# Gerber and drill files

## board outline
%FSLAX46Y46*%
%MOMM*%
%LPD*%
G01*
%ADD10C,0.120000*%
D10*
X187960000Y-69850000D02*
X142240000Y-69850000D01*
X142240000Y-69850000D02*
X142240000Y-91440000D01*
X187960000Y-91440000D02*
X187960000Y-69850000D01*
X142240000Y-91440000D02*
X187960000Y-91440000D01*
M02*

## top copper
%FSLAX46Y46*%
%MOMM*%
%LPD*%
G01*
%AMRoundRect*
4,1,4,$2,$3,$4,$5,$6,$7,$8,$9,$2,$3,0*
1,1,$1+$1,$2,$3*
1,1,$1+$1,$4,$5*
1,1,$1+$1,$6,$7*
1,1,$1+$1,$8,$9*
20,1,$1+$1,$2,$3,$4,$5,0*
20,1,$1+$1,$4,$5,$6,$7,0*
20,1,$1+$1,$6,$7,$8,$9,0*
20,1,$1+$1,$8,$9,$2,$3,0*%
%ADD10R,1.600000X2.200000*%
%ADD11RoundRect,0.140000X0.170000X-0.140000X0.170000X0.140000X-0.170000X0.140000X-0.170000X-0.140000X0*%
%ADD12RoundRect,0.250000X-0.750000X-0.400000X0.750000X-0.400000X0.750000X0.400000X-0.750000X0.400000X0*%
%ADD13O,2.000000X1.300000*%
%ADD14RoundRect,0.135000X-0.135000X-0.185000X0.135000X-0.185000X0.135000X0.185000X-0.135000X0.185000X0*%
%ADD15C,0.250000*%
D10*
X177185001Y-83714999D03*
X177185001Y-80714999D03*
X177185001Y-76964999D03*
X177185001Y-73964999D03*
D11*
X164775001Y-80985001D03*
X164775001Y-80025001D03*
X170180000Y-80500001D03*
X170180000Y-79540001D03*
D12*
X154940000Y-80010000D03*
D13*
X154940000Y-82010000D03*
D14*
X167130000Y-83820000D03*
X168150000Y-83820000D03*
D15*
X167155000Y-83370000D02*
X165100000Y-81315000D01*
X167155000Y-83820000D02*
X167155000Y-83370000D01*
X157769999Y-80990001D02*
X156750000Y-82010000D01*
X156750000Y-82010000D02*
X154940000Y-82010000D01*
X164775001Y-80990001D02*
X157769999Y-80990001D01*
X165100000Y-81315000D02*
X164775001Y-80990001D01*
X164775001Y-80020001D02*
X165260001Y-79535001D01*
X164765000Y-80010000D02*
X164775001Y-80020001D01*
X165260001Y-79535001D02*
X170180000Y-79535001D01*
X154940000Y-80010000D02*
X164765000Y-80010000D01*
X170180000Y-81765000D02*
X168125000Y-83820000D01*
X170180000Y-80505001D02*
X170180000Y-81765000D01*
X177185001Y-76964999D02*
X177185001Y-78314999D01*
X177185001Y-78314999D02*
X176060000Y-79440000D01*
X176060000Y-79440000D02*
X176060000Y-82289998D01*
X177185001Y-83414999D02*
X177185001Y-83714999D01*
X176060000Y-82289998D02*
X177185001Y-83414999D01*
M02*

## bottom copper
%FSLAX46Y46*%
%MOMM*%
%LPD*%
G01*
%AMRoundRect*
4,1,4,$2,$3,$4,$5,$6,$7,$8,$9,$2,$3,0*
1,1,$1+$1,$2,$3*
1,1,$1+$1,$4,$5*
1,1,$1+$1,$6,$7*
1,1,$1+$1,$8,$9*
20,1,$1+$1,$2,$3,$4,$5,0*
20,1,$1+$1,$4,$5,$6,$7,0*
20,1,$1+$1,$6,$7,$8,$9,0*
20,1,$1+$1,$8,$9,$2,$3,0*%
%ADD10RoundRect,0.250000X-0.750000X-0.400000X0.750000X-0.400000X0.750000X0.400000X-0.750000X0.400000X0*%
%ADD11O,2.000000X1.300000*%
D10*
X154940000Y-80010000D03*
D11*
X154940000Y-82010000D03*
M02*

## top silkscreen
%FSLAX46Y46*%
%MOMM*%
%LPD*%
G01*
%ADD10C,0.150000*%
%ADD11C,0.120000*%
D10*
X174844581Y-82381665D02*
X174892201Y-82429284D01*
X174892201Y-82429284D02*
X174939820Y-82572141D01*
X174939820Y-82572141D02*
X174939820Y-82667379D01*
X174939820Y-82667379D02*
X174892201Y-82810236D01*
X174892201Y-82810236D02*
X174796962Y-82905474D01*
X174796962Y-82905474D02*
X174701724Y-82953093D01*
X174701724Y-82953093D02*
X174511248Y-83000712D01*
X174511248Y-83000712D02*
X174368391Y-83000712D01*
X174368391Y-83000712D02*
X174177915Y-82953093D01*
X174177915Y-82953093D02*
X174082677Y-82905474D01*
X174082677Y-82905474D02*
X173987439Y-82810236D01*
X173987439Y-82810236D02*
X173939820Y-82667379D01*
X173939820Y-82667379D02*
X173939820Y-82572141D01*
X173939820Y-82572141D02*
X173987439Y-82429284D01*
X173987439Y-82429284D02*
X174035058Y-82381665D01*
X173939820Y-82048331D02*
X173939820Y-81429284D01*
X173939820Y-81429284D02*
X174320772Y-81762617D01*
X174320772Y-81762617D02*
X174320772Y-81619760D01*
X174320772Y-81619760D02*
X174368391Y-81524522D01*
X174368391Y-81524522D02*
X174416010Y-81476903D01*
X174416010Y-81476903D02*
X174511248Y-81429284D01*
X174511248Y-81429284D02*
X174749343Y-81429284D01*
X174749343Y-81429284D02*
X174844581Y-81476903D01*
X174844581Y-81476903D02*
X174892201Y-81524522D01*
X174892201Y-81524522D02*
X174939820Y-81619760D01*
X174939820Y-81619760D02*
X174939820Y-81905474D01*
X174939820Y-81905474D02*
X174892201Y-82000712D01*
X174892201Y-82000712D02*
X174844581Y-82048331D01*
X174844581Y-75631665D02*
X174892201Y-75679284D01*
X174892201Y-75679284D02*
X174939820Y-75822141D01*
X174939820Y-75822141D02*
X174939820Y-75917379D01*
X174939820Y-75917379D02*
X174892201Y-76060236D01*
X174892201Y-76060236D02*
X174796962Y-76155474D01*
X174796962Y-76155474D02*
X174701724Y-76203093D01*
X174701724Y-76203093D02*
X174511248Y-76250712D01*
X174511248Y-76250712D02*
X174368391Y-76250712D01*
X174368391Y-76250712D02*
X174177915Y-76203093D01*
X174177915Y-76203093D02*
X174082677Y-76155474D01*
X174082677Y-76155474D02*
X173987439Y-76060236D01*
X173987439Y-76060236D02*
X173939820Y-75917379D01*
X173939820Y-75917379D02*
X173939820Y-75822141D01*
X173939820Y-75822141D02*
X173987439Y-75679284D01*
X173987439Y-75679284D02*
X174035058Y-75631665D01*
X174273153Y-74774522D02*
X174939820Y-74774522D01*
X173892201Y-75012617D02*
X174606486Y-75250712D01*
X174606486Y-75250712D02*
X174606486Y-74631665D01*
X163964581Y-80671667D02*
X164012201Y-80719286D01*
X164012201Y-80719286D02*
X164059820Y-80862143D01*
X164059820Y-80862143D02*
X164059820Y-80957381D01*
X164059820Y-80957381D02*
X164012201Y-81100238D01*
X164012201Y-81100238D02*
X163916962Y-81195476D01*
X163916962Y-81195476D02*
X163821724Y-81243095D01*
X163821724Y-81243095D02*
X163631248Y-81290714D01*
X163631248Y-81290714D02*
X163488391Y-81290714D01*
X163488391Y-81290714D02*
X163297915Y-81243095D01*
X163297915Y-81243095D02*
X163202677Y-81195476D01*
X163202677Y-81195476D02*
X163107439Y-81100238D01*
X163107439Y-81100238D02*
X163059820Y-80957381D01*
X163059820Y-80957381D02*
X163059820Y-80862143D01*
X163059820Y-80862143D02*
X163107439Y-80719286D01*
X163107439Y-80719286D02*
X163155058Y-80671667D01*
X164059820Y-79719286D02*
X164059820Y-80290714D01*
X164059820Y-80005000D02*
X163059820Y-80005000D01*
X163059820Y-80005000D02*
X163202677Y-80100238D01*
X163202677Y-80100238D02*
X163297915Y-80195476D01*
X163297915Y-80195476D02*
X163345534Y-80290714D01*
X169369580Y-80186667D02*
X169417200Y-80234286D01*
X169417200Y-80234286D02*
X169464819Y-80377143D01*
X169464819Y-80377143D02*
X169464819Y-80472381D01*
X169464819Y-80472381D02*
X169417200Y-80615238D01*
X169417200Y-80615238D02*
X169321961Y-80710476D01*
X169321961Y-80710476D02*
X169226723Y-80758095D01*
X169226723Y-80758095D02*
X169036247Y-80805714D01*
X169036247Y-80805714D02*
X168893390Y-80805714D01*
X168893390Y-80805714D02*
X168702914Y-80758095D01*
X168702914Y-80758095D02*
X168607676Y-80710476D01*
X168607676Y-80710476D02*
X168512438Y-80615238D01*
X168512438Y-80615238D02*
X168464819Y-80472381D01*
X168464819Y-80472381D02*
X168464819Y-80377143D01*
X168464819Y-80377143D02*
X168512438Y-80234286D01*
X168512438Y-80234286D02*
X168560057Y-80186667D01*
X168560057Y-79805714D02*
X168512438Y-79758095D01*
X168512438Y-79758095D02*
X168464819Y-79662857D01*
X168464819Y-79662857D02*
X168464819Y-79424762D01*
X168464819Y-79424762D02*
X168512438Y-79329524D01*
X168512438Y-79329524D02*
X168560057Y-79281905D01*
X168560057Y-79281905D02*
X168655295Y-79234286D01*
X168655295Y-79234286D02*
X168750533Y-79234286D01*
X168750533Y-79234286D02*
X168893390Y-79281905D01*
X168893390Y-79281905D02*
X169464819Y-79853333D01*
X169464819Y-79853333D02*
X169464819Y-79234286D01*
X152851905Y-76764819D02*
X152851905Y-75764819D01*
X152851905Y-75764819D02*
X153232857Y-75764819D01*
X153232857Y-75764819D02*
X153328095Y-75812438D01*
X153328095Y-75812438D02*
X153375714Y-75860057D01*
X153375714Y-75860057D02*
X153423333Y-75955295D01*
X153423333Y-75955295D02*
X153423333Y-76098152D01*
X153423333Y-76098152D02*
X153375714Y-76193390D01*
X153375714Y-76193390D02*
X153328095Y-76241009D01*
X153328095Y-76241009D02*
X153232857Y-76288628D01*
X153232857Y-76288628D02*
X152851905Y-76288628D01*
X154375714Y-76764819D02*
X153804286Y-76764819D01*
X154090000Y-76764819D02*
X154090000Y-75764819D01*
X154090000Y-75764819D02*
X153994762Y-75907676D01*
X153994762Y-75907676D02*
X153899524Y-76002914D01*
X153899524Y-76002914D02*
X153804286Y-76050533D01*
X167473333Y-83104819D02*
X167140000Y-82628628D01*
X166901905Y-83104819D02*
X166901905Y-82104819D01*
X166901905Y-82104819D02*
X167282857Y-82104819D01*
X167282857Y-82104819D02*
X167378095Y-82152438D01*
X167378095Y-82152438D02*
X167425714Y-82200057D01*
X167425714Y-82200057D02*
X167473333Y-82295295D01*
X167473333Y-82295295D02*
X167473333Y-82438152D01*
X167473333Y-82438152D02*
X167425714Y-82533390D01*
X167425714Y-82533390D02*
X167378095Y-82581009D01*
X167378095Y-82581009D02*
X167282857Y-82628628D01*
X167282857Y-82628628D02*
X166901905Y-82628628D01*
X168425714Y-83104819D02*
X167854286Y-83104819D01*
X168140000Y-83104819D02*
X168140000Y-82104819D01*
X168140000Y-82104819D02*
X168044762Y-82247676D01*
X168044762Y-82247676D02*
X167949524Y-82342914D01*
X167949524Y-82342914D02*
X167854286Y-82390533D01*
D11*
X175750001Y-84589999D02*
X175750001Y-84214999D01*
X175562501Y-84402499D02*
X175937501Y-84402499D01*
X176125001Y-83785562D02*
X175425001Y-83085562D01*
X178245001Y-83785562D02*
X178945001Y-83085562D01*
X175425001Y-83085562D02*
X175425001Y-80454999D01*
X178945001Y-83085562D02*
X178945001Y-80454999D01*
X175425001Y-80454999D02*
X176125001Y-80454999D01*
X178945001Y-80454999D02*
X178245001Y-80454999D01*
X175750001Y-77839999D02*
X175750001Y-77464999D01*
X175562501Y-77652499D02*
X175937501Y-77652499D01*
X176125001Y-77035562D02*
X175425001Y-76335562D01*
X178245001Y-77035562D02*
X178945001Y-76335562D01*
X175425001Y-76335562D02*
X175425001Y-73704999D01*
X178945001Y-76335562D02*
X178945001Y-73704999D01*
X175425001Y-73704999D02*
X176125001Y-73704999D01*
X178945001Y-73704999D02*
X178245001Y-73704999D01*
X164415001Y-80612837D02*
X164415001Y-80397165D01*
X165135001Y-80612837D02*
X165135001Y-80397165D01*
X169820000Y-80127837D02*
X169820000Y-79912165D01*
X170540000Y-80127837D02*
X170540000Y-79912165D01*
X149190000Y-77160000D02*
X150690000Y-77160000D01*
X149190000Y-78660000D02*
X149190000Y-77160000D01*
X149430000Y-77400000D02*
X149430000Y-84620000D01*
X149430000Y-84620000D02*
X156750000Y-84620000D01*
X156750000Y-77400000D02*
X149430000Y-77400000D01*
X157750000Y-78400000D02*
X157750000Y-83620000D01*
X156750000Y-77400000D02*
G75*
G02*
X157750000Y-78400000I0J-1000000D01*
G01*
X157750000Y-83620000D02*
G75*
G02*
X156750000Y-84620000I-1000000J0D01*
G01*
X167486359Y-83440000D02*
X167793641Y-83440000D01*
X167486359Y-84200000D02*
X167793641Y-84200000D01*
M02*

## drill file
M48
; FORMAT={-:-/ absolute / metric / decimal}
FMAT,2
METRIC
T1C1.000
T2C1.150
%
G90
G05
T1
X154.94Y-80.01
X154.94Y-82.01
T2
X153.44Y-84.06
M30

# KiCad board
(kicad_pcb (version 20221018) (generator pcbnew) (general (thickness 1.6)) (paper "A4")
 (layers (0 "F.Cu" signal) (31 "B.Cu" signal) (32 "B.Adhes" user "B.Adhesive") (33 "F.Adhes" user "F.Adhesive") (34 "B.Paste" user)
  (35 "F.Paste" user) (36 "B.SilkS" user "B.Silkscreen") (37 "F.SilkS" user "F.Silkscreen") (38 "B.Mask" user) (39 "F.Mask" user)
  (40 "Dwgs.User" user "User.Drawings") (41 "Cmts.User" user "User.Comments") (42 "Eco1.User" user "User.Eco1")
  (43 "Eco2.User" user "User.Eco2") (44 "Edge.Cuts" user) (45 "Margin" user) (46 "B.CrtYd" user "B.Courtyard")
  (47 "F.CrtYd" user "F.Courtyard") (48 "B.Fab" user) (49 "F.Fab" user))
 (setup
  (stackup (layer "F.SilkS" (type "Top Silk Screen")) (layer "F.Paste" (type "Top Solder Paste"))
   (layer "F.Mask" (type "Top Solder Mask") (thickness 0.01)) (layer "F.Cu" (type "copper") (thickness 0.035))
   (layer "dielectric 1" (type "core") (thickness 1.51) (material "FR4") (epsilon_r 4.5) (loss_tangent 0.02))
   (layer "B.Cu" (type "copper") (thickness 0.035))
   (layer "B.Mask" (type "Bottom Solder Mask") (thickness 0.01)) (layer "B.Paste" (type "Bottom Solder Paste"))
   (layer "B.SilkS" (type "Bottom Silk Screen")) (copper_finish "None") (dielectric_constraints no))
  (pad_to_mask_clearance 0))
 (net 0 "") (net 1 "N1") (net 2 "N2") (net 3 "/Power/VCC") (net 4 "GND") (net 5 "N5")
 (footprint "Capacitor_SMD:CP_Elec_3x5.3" (layer "F.Cu") (at 177.185001 82.214999 90)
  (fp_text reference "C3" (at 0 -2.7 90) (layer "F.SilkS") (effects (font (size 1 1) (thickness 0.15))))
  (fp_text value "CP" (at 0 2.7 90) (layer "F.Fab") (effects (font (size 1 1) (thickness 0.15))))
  (fp_line (start -2.375 -1.435) (end -2 -1.435) (stroke (width 0.12) (type solid)) (layer "F.SilkS"))
  (fp_line (start -2.1875 -1.6225) (end -2.1875 -1.2475) (stroke (width 0.12) (type solid)) (layer "F.SilkS"))
  (fp_line (start -1.570563 -1.06) (end -0.870563 -1.76) (stroke (width 0.12) (type solid)) (layer "F.SilkS"))
  (fp_line (start -1.570563 1.06) (end -0.870563 1.76) (stroke (width 0.12) (type solid)) (layer "F.SilkS"))
  (fp_line (start -0.870563 -1.76) (end 1.76 -1.76) (stroke (width 0.12) (type solid)) (layer "F.SilkS"))
  (fp_line (start -0.870563 1.76) (end 1.76 1.76) (stroke (width 0.12) (type solid)) (layer "F.SilkS"))
  (fp_line (start 1.76 -1.76) (end 1.76 -1.06) (stroke (width 0.12) (type solid)) (layer "F.SilkS"))
  (fp_line (start 1.76 1.76) (end 1.76 1.06) (stroke (width 0.12) (type solid)) (layer "F.SilkS"))
  (pad "1" smd rect (at -1.5 0 90) (size 2.2 1.6) (layers "F.Cu" "F.Paste" "F.Mask") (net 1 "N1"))
  (pad "2" smd rect (at 1.5 0 90) (size 2.2 1.6) (layers "F.Cu" "F.Paste" "F.Mask") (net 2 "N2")))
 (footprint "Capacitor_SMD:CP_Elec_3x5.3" (layer "F.Cu") (at 177.185001 75.464999 90)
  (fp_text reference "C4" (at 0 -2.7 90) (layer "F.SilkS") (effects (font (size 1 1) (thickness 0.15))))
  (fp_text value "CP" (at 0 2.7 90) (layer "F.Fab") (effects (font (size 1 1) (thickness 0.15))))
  (fp_line (start -2.375 -1.435) (end -2 -1.435) (stroke (width 0.12) (type solid)) (layer "F.SilkS"))
  (fp_line (start -2.1875 -1.6225) (end -2.1875 -1.2475) (stroke (width 0.12) (type solid)) (layer "F.SilkS"))
  (fp_line (start -1.570563 -1.06) (end -0.870563 -1.76) (stroke (width 0.12) (type solid)) (layer "F.SilkS"))
  (fp_line (start -1.570563 1.06) (end -0.870563 1.76) (stroke (width 0.12) (type solid)) (layer "F.SilkS"))
  (fp_line (start -0.870563 -1.76) (end 1.76 -1.76) (stroke (width 0.12) (type solid)) (layer "F.SilkS"))
  (fp_line (start -0.870563 1.76) (end 1.76 1.76) (stroke (width 0.12) (type solid)) (layer "F.SilkS"))
  (fp_line (start 1.76 -1.76) (end 1.76 -1.06) (stroke (width 0.12) (type solid)) (layer "F.SilkS"))
  (fp_line (start 1.76 1.76) (end 1.76 1.06) (stroke (width 0.12) (type solid)) (layer "F.SilkS"))
  (pad "1" smd rect (at -1.5 0 90) (size 2.2 1.6) (layers "F.Cu" "F.Paste" "F.Mask") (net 1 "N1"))
  (pad "2" smd rect (at 1.5 0 90) (size 2.2 1.6) (layers "F.Cu" "F.Paste" "F.Mask") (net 2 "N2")))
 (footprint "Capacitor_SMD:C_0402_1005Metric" (layer "F.Cu") (at 164.775001 80.505001 90)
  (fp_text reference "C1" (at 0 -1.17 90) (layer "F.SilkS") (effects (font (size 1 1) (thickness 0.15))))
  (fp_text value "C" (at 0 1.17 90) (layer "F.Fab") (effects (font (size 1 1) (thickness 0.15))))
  (fp_line (start -0.107836 -0.36) (end 0.107836 -0.36) (stroke (width 0.12) (type solid)) (layer "F.SilkS"))
  (fp_line (start -0.107836 0.36) (end 0.107836 0.36) (stroke (width 0.12) (type solid)) (layer "F.SilkS"))
  (pad "1" smd roundrect (at -0.48 0 90) (size 0.56 0.62) (layers "F.Cu" "F.Paste" "F.Mask") (roundrect_rratio 0.25) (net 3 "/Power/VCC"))
  (pad "2" smd roundrect (at 0.48 0 90) (size 0.56 0.62) (layers "F.Cu" "F.Paste" "F.Mask") (roundrect_rratio 0.25) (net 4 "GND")))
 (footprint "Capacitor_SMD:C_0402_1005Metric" (layer "F.Cu") (at 170.18 80.020001 90)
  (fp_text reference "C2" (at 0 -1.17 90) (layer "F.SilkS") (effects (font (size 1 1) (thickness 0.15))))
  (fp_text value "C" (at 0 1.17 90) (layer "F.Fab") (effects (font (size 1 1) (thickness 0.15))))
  (fp_line (start -0.107836 -0.36) (end 0.107836 -0.36) (stroke (width 0.12) (type solid)) (layer "F.SilkS"))
  (fp_line (start -0.107836 0.36) (end 0.107836 0.36) (stroke (width 0.12) (type solid)) (layer "F.SilkS"))
  (pad "1" smd roundrect (at -0.48 0 90) (size 0.56 0.62) (layers "F.Cu" "F.Paste" "F.Mask") (roundrect_rratio 0.25) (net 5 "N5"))
  (pad "2" smd roundrect (at 0.48 0 90) (size 0.56 0.62) (layers "F.Cu" "F.Paste" "F.Mask") (roundrect_rratio 0.25) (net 4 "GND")))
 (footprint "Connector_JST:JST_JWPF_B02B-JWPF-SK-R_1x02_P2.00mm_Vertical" (layer "F.Cu") (at 154.94 80.01)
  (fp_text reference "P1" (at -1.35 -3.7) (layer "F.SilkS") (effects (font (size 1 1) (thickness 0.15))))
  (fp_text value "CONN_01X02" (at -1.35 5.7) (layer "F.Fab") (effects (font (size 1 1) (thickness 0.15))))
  (fp_line (start -5.75 -2.85) (end -4.25 -2.85) (stroke (width 0.12) (type solid)) (layer "F.SilkS"))
  (fp_line (start -5.75 -1.35) (end -5.75 -2.85) (stroke (width 0.12) (type solid)) (layer "F.SilkS"))
  (fp_line (start -5.51 -2.61) (end -5.51 4.61) (stroke (width 0.12) (type solid)) (layer "F.SilkS"))
  (fp_line (start -5.51 4.61) (end 1.81 4.61) (stroke (width 0.12) (type solid)) (layer "F.SilkS"))
  (fp_line (start 1.81 -2.61) (end -5.51 -2.61) (stroke (width 0.12) (type solid)) (layer "F.SilkS"))
  (fp_line (start 2.81 -1.61) (end 2.81 3.61) (stroke (width 0.12) (type solid)) (layer "F.SilkS"))
  (fp_arc (start 1.81 -2.61) (mid 2.517107 -2.317107) (end 2.81 -1.61) (stroke (width 0.12) (type solid)) (layer "F.SilkS"))
  (fp_arc (start 2.81 3.61) (mid 2.517107 4.317107) (end 1.81 4.61) (stroke (width 0.12) (type solid)) (layer "F.SilkS"))
  (pad "" np_thru_hole circle (at -1.5 4.05) (size 1.15 1.15) (drill 1.15) (layers "*.Cu" "*.Mask"))
  (pad "1" thru_hole roundrect (at 0 0) (size 2 1.3) (drill 1) (layers "*.Cu" "*.Mask") (roundrect_rratio 0.192308) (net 4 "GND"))
  (pad "2" thru_hole oval (at 0 2) (size 2 1.3) (drill 1) (layers "*.Cu" "*.Mask") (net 3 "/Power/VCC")))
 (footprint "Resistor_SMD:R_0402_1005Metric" (layer "F.Cu") (at 167.64 83.82)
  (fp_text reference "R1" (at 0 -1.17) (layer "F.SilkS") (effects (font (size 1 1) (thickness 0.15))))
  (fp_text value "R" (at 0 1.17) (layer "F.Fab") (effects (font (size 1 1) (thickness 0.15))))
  (fp_line (start -0.153641 -0.38) (end 0.153641 -0.38) (stroke (width 0.12) (type solid)) (layer "F.SilkS"))
  (fp_line (start -0.153641 0.38) (end 0.153641 0.38) (stroke (width 0.12) (type solid)) (layer "F.SilkS"))
  (pad "1" smd roundrect (at -0.51 0) (size 0.54 0.64) (layers "F.Cu" "F.Paste" "F.Mask") (roundrect_rratio 0.25) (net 3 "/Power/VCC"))
  (pad "2" smd roundrect (at 0.51 0) (size 0.54 0.64) (layers "F.Cu" "F.Paste" "F.Mask") (roundrect_rratio 0.25) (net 5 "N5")))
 (gr_line (start 187.96 69.85) (end 142.24 69.85) (stroke (width 0.12) (type solid)) (layer "Edge.Cuts"))
 (gr_line (start 142.24 69.85) (end 142.24 91.44) (stroke (width 0.12) (type solid)) (layer "Edge.Cuts"))
 (gr_line (start 187.96 91.44) (end 187.96 69.85) (stroke (width 0.12) (type solid)) (layer "Edge.Cuts"))
 (gr_line (start 142.24 91.44) (end 187.96 91.44) (stroke (width 0.12) (type solid)) (layer "Edge.Cuts"))
 (segment (start 167.155 83.37) (end 165.1 81.315) (width 0.25) (layer "F.Cu") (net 3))
 (segment (start 167.155 83.82) (end 167.155 83.37) (width 0.25) (layer "F.Cu") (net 3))
 (segment (start 157.769999 80.990001) (end 156.75 82.01) (width 0.25) (layer "F.Cu") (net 3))
 (segment (start 156.75 82.01) (end 154.94 82.01) (width 0.25) (layer "F.Cu") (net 3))
 (segment (start 164.775001 80.990001) (end 157.769999 80.990001) (width 0.25) (layer "F.Cu") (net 3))
 (segment (start 165.1 81.315) (end 164.775001 80.990001) (width 0.25) (layer "F.Cu") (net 3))
 (segment (start 164.775001 80.020001) (end 165.260001 79.535001) (width 0.25) (layer "F.Cu") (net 4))
 (segment (start 164.765 80.01) (end 164.775001 80.020001) (width 0.25) (layer "F.Cu") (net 4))
 (segment (start 165.260001 79.535001) (end 170.18 79.535001) (width 0.25) (layer "F.Cu") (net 4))
 (segment (start 154.94 80.01) (end 164.765 80.01) (width 0.25) (layer "F.Cu") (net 4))
 (segment (start 170.18 81.765) (end 168.125 83.82) (width 0.25) (layer "F.Cu") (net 5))
 (segment (start 170.18 80.505001) (end 170.18 81.765) (width 0.25) (layer "F.Cu") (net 5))
 (segment (start 177.185001 76.964999) (end 177.185001 78.314999) (width 0.25) (layer "F.Cu") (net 1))
 (segment (start 177.185001 78.314999) (end 176.06 79.44) (width 0.25) (layer "F.Cu") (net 1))
 (segment (start 176.06 79.44) (end 176.06 82.289998) (width 0.25) (layer "F.Cu") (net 1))
 (segment (start 177.185001 83.414999) (end 177.185001 83.714999) (width 0.25) (layer "F.Cu") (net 1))
 (segment (start 176.06 82.289998) (end 177.185001 83.414999) (width 0.25) (layer "F.Cu") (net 1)))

